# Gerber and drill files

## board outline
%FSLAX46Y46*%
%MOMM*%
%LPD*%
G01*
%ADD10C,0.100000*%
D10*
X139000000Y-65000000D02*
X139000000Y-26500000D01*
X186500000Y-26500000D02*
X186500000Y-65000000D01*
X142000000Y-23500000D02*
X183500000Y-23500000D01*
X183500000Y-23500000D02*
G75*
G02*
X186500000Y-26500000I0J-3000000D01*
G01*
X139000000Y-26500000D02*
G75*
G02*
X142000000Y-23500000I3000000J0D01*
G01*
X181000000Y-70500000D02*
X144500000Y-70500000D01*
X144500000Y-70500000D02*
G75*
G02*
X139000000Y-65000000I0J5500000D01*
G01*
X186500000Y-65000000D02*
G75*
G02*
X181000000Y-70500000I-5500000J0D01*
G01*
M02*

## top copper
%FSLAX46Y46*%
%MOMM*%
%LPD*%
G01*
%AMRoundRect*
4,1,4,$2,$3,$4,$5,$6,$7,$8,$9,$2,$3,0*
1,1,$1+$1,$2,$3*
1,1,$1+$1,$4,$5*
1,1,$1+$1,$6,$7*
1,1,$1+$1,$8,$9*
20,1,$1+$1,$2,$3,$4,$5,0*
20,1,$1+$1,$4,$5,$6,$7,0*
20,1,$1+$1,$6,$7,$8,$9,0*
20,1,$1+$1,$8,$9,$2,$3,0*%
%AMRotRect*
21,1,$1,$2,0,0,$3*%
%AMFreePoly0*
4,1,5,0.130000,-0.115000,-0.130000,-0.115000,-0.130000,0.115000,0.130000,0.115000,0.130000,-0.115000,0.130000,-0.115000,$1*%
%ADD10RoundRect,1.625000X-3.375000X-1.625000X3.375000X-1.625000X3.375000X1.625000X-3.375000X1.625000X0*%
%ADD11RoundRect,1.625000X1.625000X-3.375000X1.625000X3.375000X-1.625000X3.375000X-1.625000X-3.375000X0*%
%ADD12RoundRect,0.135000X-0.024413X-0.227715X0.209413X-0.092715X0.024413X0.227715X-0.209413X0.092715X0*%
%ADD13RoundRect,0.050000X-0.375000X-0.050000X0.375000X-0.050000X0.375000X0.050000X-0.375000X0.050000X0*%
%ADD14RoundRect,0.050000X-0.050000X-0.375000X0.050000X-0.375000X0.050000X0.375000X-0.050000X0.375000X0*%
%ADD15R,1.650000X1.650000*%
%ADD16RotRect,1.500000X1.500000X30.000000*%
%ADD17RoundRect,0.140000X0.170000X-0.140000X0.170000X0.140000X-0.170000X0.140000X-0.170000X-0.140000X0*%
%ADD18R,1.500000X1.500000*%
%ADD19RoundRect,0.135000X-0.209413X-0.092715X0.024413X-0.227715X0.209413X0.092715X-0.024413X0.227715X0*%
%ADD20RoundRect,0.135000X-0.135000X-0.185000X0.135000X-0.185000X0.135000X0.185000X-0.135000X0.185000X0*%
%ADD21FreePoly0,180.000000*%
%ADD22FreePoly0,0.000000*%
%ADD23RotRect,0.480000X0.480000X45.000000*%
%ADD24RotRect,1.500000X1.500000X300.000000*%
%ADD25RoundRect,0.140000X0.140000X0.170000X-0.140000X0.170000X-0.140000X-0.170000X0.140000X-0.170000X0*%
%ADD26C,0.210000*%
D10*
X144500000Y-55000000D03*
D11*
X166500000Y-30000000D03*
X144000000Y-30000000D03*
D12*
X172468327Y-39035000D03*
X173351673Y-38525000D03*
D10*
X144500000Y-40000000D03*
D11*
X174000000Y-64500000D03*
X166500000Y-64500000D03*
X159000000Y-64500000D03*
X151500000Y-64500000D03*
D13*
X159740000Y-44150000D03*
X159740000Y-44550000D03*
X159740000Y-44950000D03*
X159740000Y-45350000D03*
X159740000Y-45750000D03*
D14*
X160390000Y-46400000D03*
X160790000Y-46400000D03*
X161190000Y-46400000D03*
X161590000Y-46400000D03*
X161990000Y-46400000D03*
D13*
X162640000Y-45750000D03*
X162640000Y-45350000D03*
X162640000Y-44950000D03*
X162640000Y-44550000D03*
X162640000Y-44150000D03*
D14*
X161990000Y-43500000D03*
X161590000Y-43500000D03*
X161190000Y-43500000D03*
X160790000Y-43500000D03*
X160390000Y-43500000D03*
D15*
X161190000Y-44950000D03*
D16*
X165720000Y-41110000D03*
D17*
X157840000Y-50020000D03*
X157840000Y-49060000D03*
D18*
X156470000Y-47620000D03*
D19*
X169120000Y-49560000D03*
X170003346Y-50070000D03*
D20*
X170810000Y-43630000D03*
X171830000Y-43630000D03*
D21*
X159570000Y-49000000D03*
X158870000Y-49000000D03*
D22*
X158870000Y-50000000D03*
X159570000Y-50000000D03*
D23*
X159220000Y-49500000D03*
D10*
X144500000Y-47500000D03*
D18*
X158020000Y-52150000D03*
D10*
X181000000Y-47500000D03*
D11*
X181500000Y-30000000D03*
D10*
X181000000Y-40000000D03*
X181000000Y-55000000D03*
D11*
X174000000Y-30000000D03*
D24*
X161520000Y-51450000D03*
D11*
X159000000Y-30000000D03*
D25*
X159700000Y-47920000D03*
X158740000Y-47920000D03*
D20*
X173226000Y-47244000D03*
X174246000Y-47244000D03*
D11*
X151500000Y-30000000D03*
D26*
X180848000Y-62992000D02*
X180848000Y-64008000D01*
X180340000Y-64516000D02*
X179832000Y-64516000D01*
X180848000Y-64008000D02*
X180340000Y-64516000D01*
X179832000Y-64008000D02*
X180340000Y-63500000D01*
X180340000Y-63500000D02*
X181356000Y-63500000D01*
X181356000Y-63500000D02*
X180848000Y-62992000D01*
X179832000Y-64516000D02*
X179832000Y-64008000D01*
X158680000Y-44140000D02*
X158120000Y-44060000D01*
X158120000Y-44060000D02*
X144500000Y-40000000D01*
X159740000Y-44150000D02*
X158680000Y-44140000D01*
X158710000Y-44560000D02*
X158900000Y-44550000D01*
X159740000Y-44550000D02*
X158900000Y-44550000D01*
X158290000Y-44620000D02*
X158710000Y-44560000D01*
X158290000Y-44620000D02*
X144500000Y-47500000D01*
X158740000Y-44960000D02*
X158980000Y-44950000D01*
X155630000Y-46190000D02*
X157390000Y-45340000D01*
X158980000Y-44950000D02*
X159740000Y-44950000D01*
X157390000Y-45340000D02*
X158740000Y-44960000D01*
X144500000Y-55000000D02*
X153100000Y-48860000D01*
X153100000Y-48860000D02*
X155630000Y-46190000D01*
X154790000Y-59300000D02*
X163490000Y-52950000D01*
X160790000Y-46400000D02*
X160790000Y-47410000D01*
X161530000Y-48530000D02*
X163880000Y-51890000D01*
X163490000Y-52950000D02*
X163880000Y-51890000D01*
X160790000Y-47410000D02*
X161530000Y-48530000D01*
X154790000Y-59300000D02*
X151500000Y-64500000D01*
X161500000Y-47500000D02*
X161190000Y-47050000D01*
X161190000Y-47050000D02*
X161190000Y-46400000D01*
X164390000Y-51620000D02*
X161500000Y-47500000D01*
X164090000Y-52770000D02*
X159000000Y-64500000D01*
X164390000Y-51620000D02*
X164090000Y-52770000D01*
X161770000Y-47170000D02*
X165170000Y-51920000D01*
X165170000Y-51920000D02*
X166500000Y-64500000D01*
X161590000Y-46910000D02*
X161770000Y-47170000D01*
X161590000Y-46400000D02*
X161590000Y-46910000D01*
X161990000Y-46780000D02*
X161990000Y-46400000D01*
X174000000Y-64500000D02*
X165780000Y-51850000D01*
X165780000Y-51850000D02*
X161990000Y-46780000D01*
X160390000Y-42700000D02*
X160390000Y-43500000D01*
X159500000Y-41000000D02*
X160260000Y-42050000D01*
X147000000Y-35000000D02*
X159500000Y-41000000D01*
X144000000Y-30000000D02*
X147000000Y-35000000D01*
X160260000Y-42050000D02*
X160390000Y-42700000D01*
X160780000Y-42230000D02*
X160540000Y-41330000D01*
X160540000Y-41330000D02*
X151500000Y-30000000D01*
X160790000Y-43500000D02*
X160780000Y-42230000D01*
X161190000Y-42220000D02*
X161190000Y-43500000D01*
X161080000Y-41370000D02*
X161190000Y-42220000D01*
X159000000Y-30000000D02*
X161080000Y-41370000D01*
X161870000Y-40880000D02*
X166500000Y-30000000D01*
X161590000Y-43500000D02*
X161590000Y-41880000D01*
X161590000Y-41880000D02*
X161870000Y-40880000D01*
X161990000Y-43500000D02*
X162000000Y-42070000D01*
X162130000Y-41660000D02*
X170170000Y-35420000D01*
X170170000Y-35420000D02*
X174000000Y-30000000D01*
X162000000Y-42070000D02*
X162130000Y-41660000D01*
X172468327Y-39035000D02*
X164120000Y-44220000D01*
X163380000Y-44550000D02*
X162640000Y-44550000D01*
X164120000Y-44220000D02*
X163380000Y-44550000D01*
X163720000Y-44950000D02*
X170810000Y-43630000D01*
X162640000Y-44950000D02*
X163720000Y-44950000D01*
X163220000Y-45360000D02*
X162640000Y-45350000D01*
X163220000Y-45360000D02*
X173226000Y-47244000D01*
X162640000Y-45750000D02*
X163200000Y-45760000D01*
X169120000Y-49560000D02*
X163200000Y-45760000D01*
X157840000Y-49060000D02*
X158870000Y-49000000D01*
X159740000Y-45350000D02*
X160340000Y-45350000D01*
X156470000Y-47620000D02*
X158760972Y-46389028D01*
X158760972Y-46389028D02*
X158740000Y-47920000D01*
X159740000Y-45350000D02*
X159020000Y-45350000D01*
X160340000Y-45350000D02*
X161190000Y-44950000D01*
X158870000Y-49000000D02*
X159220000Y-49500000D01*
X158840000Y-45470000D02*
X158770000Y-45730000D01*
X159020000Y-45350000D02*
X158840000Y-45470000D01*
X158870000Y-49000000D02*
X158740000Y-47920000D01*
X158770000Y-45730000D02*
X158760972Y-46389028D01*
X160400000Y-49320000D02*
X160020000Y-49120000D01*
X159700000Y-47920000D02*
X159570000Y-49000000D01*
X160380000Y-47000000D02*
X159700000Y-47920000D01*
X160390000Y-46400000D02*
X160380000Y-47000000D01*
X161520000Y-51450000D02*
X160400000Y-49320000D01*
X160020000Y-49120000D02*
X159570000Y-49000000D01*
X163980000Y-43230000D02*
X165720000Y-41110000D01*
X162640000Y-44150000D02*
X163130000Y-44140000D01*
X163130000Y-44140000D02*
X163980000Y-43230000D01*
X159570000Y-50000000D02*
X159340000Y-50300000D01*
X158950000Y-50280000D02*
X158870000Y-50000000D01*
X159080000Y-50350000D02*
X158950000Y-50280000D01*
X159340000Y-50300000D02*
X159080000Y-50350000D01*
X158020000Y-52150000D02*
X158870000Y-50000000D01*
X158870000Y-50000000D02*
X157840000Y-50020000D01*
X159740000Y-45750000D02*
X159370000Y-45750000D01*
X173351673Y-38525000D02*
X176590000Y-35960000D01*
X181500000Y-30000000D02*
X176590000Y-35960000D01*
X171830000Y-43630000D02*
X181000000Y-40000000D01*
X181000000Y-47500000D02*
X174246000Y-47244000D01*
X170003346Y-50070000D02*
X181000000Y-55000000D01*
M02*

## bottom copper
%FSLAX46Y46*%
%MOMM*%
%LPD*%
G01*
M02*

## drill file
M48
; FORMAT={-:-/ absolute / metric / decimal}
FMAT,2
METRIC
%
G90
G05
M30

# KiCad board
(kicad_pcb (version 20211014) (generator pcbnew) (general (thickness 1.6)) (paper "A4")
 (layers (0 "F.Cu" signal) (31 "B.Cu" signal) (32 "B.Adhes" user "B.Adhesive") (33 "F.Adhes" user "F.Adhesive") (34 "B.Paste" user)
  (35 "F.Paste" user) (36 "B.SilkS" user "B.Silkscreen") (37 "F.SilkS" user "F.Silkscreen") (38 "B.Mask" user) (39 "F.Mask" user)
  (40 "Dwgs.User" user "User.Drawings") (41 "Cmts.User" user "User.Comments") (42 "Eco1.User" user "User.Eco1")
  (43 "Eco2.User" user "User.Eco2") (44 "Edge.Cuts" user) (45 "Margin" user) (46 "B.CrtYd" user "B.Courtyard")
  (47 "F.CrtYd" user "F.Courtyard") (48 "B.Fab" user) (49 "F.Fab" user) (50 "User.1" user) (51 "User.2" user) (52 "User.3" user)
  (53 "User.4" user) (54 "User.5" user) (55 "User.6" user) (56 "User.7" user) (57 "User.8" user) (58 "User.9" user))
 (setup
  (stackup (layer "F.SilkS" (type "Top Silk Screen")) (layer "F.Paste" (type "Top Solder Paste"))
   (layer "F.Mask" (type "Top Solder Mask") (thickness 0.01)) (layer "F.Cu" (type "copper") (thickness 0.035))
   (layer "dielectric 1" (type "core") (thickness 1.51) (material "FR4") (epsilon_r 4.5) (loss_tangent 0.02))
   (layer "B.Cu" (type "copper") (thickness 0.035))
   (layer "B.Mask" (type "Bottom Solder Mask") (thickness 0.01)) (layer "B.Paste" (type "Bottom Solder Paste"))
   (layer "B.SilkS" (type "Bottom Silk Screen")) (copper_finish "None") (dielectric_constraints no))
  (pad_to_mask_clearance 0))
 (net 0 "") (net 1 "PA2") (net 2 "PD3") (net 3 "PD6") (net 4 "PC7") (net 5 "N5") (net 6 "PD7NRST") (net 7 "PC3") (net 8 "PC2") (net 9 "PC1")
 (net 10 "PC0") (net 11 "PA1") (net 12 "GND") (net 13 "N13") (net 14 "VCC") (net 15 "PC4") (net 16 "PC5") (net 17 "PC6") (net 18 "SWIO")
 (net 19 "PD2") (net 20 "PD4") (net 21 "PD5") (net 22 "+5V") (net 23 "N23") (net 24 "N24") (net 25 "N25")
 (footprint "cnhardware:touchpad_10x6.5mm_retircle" (layer "F.Cu") (at 144.5 55)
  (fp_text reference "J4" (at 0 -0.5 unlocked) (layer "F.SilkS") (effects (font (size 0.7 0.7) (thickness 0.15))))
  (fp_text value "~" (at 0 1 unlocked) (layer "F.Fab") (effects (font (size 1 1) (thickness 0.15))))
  (pad "1" smd roundrect (at 0 0) (size 10 6.5) (layers "F.Cu") (roundrect_rratio 0.25) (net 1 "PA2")))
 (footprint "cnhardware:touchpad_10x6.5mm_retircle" (layer "F.Cu") (at 166.5 30 90)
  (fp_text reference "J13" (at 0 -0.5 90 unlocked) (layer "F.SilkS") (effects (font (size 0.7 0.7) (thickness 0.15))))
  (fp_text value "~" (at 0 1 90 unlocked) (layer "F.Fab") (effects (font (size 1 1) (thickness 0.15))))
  (pad "1" smd roundrect (at 0 0 90) (size 10 6.5) (layers "F.Cu") (roundrect_rratio 0.25) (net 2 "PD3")))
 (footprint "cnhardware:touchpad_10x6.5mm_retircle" (layer "F.Cu") (at 144 30 90)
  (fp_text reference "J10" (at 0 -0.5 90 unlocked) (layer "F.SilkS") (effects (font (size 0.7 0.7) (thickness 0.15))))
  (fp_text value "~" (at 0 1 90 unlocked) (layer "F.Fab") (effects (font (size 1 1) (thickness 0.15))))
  (pad "1" smd roundrect (at 0 0 90) (size 10 6.5) (layers "F.Cu") (roundrect_rratio 0.25) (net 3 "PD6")))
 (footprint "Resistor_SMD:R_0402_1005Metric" (layer "F.Cu") (at 172.91 38.78 30)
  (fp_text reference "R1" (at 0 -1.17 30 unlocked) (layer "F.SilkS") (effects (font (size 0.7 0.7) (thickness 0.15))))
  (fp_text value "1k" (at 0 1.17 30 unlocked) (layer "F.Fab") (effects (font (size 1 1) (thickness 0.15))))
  (pad "1" smd roundrect (at -0.51 0 30) (size 0.54 0.64) (layers "F.Cu" "F.Paste" "F.Mask") (roundrect_rratio 0.25) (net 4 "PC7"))
  (pad "2" smd roundrect (at 0.51 0 30) (size 0.54 0.64) (layers "F.Cu" "F.Paste" "F.Mask") (roundrect_rratio 0.25) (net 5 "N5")))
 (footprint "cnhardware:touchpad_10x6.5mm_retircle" (layer "F.Cu") (at 144.5 40)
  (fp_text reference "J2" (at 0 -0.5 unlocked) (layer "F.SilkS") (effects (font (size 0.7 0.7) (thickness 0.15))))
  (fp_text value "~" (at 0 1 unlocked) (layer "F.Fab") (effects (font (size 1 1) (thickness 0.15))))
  (pad "1" smd roundrect (at 0 0) (size 10 6.5) (layers "F.Cu") (roundrect_rratio 0.25) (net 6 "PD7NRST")))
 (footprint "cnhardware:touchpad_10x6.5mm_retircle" (layer "F.Cu") (at 174 64.5 90)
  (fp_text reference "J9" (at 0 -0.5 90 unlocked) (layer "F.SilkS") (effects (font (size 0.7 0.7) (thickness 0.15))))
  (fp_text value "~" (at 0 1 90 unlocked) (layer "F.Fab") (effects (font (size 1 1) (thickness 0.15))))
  (pad "1" smd roundrect (at 0 0 90) (size 10 6.5) (layers "F.Cu") (roundrect_rratio 0.25) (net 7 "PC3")))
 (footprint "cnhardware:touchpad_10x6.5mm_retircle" (layer "F.Cu") (at 166.5 64.5 90)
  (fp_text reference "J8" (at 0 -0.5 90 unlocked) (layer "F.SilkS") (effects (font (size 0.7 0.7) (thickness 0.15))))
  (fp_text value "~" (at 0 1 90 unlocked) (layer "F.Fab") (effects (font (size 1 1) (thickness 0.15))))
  (pad "1" smd roundrect (at 0 0 90) (size 10 6.5) (layers "F.Cu") (roundrect_rratio 0.25) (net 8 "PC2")))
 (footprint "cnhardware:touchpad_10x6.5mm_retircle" (layer "F.Cu") (at 159 64.5 90)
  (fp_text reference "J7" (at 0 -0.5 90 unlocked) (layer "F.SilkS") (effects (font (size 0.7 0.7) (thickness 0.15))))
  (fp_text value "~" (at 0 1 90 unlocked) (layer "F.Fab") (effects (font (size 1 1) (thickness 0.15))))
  (pad "1" smd roundrect (at 0 0 90) (size 10 6.5) (layers "F.Cu") (roundrect_rratio 0.25) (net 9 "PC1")))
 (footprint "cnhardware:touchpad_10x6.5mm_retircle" (layer "F.Cu") (at 151.5 64.5 90)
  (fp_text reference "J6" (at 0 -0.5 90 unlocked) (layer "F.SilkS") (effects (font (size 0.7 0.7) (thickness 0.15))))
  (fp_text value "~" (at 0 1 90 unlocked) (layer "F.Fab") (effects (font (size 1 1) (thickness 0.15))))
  (pad "1" smd roundrect (at 0 0 90) (size 10 6.5) (layers "F.Cu") (roundrect_rratio 0.25) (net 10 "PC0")))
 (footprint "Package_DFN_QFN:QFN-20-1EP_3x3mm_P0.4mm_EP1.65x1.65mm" (layer "F.Cu") (at 161.19 44.95)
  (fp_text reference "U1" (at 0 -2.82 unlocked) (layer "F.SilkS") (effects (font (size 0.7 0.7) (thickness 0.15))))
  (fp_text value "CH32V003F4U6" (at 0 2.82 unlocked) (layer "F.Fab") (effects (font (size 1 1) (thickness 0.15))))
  (pad "" smd roundrect (at 0.41 -0.41) (size 0.67 0.67) (layers "F.Paste") (roundrect_rratio 0.25))
  (pad "" smd roundrect (at -0.41 0.41) (size 0.67 0.67) (layers "F.Paste") (roundrect_rratio 0.25))
  (pad "" smd roundrect (at 0.41 0.41) (size 0.67 0.67) (layers "F.Paste") (roundrect_rratio 0.25))
  (pad "" smd roundrect (at -0.41 -0.41) (size 0.67 0.67) (layers "F.Paste") (roundrect_rratio 0.25))
  (pad "1" smd roundrect (at -1.45 -0.8) (size 0.85 0.2) (layers "F.Cu" "F.Paste" "F.Mask") (roundrect_rratio 0.25) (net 6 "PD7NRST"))
  (pad "2" smd roundrect (at -1.45 -0.4) (size 0.85 0.2) (layers "F.Cu" "F.Paste" "F.Mask") (roundrect_rratio 0.25) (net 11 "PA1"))
  (pad "3" smd roundrect (at -1.45 0) (size 0.85 0.2) (layers "F.Cu" "F.Paste" "F.Mask") (roundrect_rratio 0.25) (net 1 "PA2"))
  (pad "4" smd roundrect (at -1.45 0.4) (size 0.85 0.2) (layers "F.Cu" "F.Paste" "F.Mask") (roundrect_rratio 0.25) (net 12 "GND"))
  (pad "5" smd roundrect (at -1.45 0.8) (size 0.85 0.2) (layers "F.Cu" "F.Paste" "F.Mask") (roundrect_rratio 0.25) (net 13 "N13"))
  (pad "6" smd roundrect (at -0.8 1.45) (size 0.2 0.85) (layers "F.Cu" "F.Paste" "F.Mask") (roundrect_rratio 0.25) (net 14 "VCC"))
  (pad "7" smd roundrect (at -0.4 1.45) (size 0.2 0.85) (layers "F.Cu" "F.Paste" "F.Mask") (roundrect_rratio 0.25) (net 10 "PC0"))
  (pad "8" smd roundrect (at 0 1.45) (size 0.2 0.85) (layers "F.Cu" "F.Paste" "F.Mask") (roundrect_rratio 0.25) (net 9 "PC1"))
  (pad "9" smd roundrect (at 0.4 1.45) (size 0.2 0.85) (layers "F.Cu" "F.Paste" "F.Mask") (roundrect_rratio 0.25) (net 8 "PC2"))
  (pad "10" smd roundrect (at 0.8 1.45) (size 0.2 0.85) (layers "F.Cu" "F.Paste" "F.Mask") (roundrect_rratio 0.25) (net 7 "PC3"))
  (pad "11" smd roundrect (at 1.45 0.8) (size 0.85 0.2) (layers "F.Cu" "F.Paste" "F.Mask") (roundrect_rratio 0.25) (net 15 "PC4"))
  (pad "12" smd roundrect (at 1.45 0.4) (size 0.85 0.2) (layers "F.Cu" "F.Paste" "F.Mask") (roundrect_rratio 0.25) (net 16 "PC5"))
  (pad "13" smd roundrect (at 1.45 0) (size 0.85 0.2) (layers "F.Cu" "F.Paste" "F.Mask") (roundrect_rratio 0.25) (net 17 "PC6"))
  (pad "14" smd roundrect (at 1.45 -0.4) (size 0.85 0.2) (layers "F.Cu" "F.Paste" "F.Mask") (roundrect_rratio 0.25) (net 4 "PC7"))
  (pad "15" smd roundrect (at 1.45 -0.8) (size 0.85 0.2) (layers "F.Cu" "F.Paste" "F.Mask") (roundrect_rratio 0.25) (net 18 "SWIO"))
  (pad "16" smd roundrect (at 0.8 -1.45) (size 0.2 0.85) (layers "F.Cu" "F.Paste" "F.Mask") (roundrect_rratio 0.25) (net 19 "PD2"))
  (pad "17" smd roundrect (at 0.4 -1.45) (size 0.2 0.85) (layers "F.Cu" "F.Paste" "F.Mask") (roundrect_rratio 0.25) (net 2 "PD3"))
  (pad "18" smd roundrect (at 0 -1.45) (size 0.2 0.85) (layers "F.Cu" "F.Paste" "F.Mask") (roundrect_rratio 0.25) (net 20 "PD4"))
  (pad "19" smd roundrect (at -0.4 -1.45) (size 0.2 0.85) (layers "F.Cu" "F.Paste" "F.Mask") (roundrect_rratio 0.25) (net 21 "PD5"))
  (pad "20" smd roundrect (at -0.8 -1.45) (size 0.2 0.85) (layers "F.Cu" "F.Paste" "F.Mask") (roundrect_rratio 0.25) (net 3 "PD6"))
  (pad "21" smd rect (at 0 0) (size 1.65 1.65) (layers "F.Cu" "F.Mask") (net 12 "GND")))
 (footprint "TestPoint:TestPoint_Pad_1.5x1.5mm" (layer "F.Cu") (at 165.72 41.11 30)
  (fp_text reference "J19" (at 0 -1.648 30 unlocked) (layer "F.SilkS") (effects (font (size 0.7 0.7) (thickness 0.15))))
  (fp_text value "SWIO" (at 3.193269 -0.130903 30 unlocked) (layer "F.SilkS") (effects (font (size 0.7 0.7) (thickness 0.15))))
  (pad "1" smd rect (at 0 0 30) (size 1.5 1.5) (layers "F.Cu" "F.Mask") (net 18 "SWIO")))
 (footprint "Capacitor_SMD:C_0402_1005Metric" (layer "F.Cu") (at 157.84 49.54 90)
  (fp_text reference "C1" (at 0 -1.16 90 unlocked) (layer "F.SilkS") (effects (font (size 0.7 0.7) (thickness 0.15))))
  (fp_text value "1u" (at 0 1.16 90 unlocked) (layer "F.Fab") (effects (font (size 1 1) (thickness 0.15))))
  (pad "1" smd roundrect (at -0.48 0 90) (size 0.56 0.62) (layers "F.Cu" "F.Paste" "F.Mask") (roundrect_rratio 0.25) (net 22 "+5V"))
  (pad "2" smd roundrect (at 0.48 0 90) (size 0.56 0.62) (layers "F.Cu" "F.Paste" "F.Mask") (roundrect_rratio 0.25) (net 12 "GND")))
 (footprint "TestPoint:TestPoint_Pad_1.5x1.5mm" (layer "F.Cu") (at 156.47 47.62)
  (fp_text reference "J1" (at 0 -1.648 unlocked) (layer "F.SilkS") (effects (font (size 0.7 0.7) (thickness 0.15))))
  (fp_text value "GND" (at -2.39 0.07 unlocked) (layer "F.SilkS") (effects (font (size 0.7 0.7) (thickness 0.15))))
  (pad "1" smd rect (at 0 0) (size 1.5 1.5) (layers "F.Cu" "F.Mask") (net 12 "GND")))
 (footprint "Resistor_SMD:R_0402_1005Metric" (layer "F.Cu") (at 169.561673 49.815 -30)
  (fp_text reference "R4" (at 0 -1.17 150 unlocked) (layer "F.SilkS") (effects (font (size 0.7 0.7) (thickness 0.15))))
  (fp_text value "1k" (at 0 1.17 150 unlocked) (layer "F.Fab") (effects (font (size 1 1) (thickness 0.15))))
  (pad "1" smd roundrect (at -0.51 0 330) (size 0.54 0.64) (layers "F.Cu" "F.Paste" "F.Mask") (roundrect_rratio 0.25) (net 15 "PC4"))
  (pad "2" smd roundrect (at 0.51 0 330) (size 0.54 0.64) (layers "F.Cu" "F.Paste" "F.Mask") (roundrect_rratio 0.25) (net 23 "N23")))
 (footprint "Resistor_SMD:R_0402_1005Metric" (layer "F.Cu") (at 171.32 43.63)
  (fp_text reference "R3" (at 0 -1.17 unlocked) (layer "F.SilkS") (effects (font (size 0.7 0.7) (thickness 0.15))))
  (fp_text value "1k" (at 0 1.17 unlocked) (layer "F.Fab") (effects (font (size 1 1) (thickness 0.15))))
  (pad "1" smd roundrect (at -0.51 0) (size 0.54 0.64) (layers "F.Cu" "F.Paste" "F.Mask") (roundrect_rratio 0.25) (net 17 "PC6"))
  (pad "2" smd roundrect (at 0.51 0) (size 0.54 0.64) (layers "F.Cu" "F.Paste" "F.Mask") (roundrect_rratio 0.25) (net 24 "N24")))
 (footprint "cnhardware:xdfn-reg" (layer "F.Cu") (at 159.22 49.5 180)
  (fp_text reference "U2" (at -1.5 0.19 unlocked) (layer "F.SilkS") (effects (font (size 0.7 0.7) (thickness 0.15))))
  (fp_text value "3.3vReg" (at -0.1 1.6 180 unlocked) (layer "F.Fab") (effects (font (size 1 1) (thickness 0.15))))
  (pad "1" smd custom (at -0.35 0.5 180) (size 0.26 0.23) (layers "F.Cu" "F.Paste" "F.Mask") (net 14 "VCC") (zone_connect 0)
   (options (clearance outline) (anchor rect)) (primitives))
  (pad "2" smd custom (at 0.35 0.5 180) (size 0.26 0.23) (layers "F.Cu" "F.Paste" "F.Mask") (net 12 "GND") (zone_connect 0)
   (options (clearance outline) (anchor rect)) (primitives))
  (pad "3" smd custom (at 0.35 -0.5) (size 0.26 0.23) (layers "F.Cu" "F.Paste" "F.Mask") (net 22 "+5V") (zone_connect 0)
   (options (clearance outline) (anchor rect)) (primitives))
  (pad "4" smd custom (at -0.35 -0.5) (size 0.26 0.23) (layers "F.Cu" "F.Paste" "F.Mask") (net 22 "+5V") (zone_connect 0)
   (options (clearance outline) (anchor rect)) (primitives))
  (pad "5" smd rect (at 0 0 45) (size 0.48 0.48) (layers "F.Cu" "F.Paste" "F.Mask") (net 12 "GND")))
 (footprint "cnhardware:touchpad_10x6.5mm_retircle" (layer "F.Cu") (at 144.5 47.5)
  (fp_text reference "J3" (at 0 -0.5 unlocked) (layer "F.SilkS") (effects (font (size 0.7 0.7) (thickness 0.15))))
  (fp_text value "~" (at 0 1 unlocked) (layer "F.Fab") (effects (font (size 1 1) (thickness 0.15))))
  (pad "1" smd roundrect (at 0 0) (size 10 6.5) (layers "F.Cu") (roundrect_rratio 0.25) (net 11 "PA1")))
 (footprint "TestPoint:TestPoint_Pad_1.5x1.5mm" (layer "F.Cu") (at 158.02 52.15 90)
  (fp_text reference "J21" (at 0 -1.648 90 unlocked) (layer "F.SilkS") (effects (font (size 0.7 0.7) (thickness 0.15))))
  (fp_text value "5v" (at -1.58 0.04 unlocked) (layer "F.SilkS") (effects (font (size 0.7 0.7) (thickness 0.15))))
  (pad "1" smd rect (at 0 0 90) (size 1.5 1.5) (layers "F.Cu" "F.Mask") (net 22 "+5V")))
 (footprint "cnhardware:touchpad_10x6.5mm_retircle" (layer "F.Cu") (at 181 47.5)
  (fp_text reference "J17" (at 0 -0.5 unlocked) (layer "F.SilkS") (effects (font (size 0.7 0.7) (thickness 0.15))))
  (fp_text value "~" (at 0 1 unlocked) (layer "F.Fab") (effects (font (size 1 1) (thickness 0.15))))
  (pad "1" smd roundrect (at 0 0) (size 10 6.5) (layers "F.Cu") (roundrect_rratio 0.25) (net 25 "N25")))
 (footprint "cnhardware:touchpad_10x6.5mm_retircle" (layer "F.Cu") (at 181.5 30 90)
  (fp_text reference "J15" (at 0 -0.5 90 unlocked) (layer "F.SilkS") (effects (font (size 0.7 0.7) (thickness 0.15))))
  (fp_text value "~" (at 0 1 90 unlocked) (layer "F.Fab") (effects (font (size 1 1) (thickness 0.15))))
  (pad "1" smd roundrect (at 0 0 90) (size 10 6.5) (layers "F.Cu") (roundrect_rratio 0.25) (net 5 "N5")))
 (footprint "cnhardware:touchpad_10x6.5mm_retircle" (layer "F.Cu") (at 181 40)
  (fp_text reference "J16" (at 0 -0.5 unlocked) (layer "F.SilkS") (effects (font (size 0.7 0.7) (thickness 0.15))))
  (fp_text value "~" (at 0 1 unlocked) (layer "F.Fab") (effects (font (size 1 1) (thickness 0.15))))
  (pad "1" smd roundrect (at 0 0) (size 10 6.5) (layers "F.Cu") (roundrect_rratio 0.25) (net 24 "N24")))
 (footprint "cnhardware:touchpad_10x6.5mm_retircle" (layer "F.Cu") (at 181 55)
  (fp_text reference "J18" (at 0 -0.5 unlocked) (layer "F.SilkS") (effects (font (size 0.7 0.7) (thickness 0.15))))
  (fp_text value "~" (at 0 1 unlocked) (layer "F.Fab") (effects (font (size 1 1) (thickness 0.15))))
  (pad "1" smd roundrect (at 0 0) (size 10 6.5) (layers "F.Cu") (roundrect_rratio 0.25) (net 23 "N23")))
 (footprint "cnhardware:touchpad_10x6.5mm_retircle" (layer "F.Cu") (at 174 30 90)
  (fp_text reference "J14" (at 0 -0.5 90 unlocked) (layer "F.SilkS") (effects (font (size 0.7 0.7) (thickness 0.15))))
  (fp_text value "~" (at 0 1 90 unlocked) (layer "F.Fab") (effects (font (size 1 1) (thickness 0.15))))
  (pad "1" smd roundrect (at 0 0 90) (size 10 6.5) (layers "F.Cu") (roundrect_rratio 0.25) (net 19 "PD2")))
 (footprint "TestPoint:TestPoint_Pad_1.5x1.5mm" (layer "F.Cu") (at 161.52 51.45 -60)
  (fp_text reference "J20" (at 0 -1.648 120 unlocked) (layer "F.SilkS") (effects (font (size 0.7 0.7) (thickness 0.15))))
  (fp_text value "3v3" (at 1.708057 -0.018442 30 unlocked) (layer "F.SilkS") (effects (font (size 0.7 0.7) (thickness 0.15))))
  (pad "1" smd rect (at 0 0 300) (size 1.5 1.5) (layers "F.Cu" "F.Mask") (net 14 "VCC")))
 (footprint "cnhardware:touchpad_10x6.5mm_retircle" (layer "F.Cu") (at 159 30 90)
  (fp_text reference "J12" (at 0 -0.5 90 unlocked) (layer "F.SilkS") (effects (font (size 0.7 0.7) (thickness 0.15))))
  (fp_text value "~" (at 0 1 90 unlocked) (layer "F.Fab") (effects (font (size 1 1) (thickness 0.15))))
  (pad "1" smd roundrect (at 0 0 90) (size 10 6.5) (layers "F.Cu") (roundrect_rratio 0.25) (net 20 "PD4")))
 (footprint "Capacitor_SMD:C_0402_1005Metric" (layer "F.Cu") (at 159.22 47.92 180)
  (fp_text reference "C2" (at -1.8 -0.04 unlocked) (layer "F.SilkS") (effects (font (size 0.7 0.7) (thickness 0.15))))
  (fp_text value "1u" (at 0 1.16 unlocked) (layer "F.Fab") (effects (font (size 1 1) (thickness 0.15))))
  (pad "1" smd roundrect (at -0.48 0 180) (size 0.56 0.62) (layers "F.Cu" "F.Paste" "F.Mask") (roundrect_rratio 0.25) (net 14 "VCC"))
  (pad "2" smd roundrect (at 0.48 0 180) (size 0.56 0.62) (layers "F.Cu" "F.Paste" "F.Mask") (roundrect_rratio 0.25) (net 12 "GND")))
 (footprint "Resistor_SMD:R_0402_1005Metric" (layer "F.Cu") (at 173.736 47.244)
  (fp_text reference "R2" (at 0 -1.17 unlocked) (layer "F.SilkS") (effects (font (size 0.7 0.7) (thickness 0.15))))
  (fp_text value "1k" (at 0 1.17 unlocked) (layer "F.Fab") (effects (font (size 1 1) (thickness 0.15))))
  (pad "1" smd roundrect (at -0.51 0) (size 0.54 0.64) (layers "F.Cu" "F.Paste" "F.Mask") (roundrect_rratio 0.25) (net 16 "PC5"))
  (pad "2" smd roundrect (at 0.51 0) (size 0.54 0.64) (layers "F.Cu" "F.Paste" "F.Mask") (roundrect_rratio 0.25) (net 25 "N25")))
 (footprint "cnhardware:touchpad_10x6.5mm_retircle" (layer "F.Cu") (at 151.5 30 90)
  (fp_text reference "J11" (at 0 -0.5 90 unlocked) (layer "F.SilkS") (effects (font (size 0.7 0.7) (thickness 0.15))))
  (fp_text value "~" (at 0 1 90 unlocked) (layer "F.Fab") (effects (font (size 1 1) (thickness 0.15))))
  (pad "1" smd roundrect (at 0 0 90) (size 10 6.5) (layers "F.Cu") (roundrect_rratio 0.25) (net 21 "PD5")))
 (gr_line (start 139 65) (end 139 26.5) (layer "Edge.Cuts") (width 0.1))
 (gr_line (start 186.5 26.5) (end 186.5 65) (layer "Edge.Cuts") (width 0.1))
 (gr_line (start 142 23.5) (end 183.5 23.5) (layer "Edge.Cuts") (width 0.1))
 (gr_arc (start 183.5 23.5) (mid 185.62132 24.37868) (end 186.5 26.5) (layer "Edge.Cuts") (width 0.1))
 (gr_arc (start 139 26.5) (mid 139.87868 24.37868) (end 142 23.5) (layer "Edge.Cuts") (width 0.1))
 (gr_line (start 181 70.5) (end 144.5 70.5) (layer "Edge.Cuts") (width 0.1))
 (gr_arc (start 144.5 70.5) (mid 140.610913 68.889087) (end 139 65) (layer "Edge.Cuts") (width 0.1))
 (gr_arc (start 186.5 65) (mid 184.889087 68.889087) (end 181 70.5) (layer "Edge.Cuts") (width 0.1))
 (segment (start 180.848 62.992) (end 180.848 64.008) (width 0.21) (layer "F.Cu") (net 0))
 (segment (start 180.34 64.516) (end 179.832 64.516) (width 0.21) (layer "F.Cu") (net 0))
 (segment (start 180.848 64.008) (end 180.34 64.516) (width 0.21) (layer "F.Cu") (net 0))
 (segment (start 179.832 64.008) (end 180.34 63.5) (width 0.21) (layer "F.Cu") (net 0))
 (segment (start 180.34 63.5) (end 181.356 63.5) (width 0.21) (layer "F.Cu") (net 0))
 (segment (start 181.356 63.5) (end 180.848 62.992) (width 0.21) (layer "F.Cu") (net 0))
 (segment (start 179.832 64.516) (end 179.832 64.008) (width 0.21) (layer "F.Cu") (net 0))
 (segment (start 158.68 44.14) (end 158.12 44.06) (width 0.21) (layer "F.Cu") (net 6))
 (segment (start 158.12 44.06) (end 144.5 40) (width 0.21) (layer "F.Cu") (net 6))
 (segment (start 159.74 44.15) (end 158.68 44.14) (width 0.21) (layer "F.Cu") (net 6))
 (segment (start 158.71 44.56) (end 158.9 44.55) (width 0.21) (layer "F.Cu") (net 11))
 (segment (start 159.74 44.55) (end 158.9 44.55) (width 0.21) (layer "F.Cu") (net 11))
 (segment (start 158.29 44.62) (end 158.71 44.56) (width 0.21) (layer "F.Cu") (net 11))
 (segment (start 158.29 44.62) (end 144.5 47.5) (width 0.21) (layer "F.Cu") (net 11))
 (segment (start 158.74 44.96) (end 158.98 44.95) (width 0.21) (layer "F.Cu") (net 1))
 (segment (start 155.63 46.19) (end 157.39 45.34) (width 0.21) (layer "F.Cu") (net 1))
 (segment (start 158.98 44.95) (end 159.74 44.95) (width 0.21) (layer "F.Cu") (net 1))
 (segment (start 157.39 45.34) (end 158.74 44.96) (width 0.21) (layer "F.Cu") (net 1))
 (segment (start 144.5 55) (end 153.1 48.86) (width 0.21) (layer "F.Cu") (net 1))
 (segment (start 153.1 48.86) (end 155.63 46.19) (width 0.21) (layer "F.Cu") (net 1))
 (segment (start 154.79 59.3) (end 163.49 52.95) (width 0.21) (layer "F.Cu") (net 10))
 (segment (start 160.79 46.4) (end 160.79 47.41) (width 0.21) (layer "F.Cu") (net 10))
 (segment (start 161.53 48.53) (end 163.88 51.89) (width 0.21) (layer "F.Cu") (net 10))
 (segment (start 163.49 52.95) (end 163.88 51.89) (width 0.21) (layer "F.Cu") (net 10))
 (segment (start 160.79 47.41) (end 161.53 48.53) (width 0.21) (layer "F.Cu") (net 10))
 (segment (start 154.79 59.3) (end 151.5 64.5) (width 0.21) (layer "F.Cu") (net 10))
 (segment (start 161.5 47.5) (end 161.19 47.05) (width 0.21) (layer "F.Cu") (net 9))
 (segment (start 161.19 47.05) (end 161.19 46.4) (width 0.21) (layer "F.Cu") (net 9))
 (segment (start 164.39 51.62) (end 161.5 47.5) (width 0.21) (layer "F.Cu") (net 9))
 (segment (start 164.09 52.77) (end 159 64.5) (width 0.21) (layer "F.Cu") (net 9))
 (segment (start 164.39 51.62) (end 164.09 52.77) (width 0.21) (layer "F.Cu") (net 9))
 (segment (start 161.77 47.17) (end 165.17 51.92) (width 0.21) (layer "F.Cu") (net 8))
 (segment (start 165.17 51.92) (end 166.5 64.5) (width 0.21) (layer "F.Cu") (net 8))
 (segment (start 161.59 46.91) (end 161.77 47.17) (width 0.21) (layer "F.Cu") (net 8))
 (segment (start 161.59 46.4) (end 161.59 46.91) (width 0.21) (layer "F.Cu") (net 8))
 (segment (start 161.99 46.78) (end 161.99 46.4) (width 0.21) (layer "F.Cu") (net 7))
 (segment (start 174 64.5) (end 165.78 51.85) (width 0.21) (layer "F.Cu") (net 7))
 (segment (start 165.78 51.85) (end 161.99 46.78) (width 0.21) (layer "F.Cu") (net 7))
 (segment (start 160.39 42.7) (end 160.39 43.5) (width 0.21) (layer "F.Cu") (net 3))
 (segment (start 159.5 41) (end 160.26 42.05) (width 0.21) (layer "F.Cu") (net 3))
 (segment (start 147 35) (end 159.5 41) (width 0.21) (layer "F.Cu") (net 3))
 (segment (start 144 30) (end 147 35) (width 0.21) (layer "F.Cu") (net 3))
 (segment (start 160.26 42.05) (end 160.39 42.7) (width 0.21) (layer "F.Cu") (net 3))
 (segment (start 160.78 42.23) (end 160.54 41.33) (width 0.21) (layer "F.Cu") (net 21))
 (segment (start 160.54 41.33) (end 151.5 30) (width 0.21) (layer "F.Cu") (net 21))
 (segment (start 160.79 43.5) (end 160.78 42.23) (width 0.21) (layer "F.Cu") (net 21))
 (segment (start 161.19 42.22) (end 161.19 43.5) (width 0.21) (layer "F.Cu") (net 20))
 (segment (start 161.08 41.37) (end 161.19 42.22) (width 0.21) (layer "F.Cu") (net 20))
 (segment (start 159 30) (end 161.08 41.37) (width 0.21) (layer "F.Cu") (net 20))
 (segment (start 161.87 40.88) (end 166.5 30) (width 0.21) (layer "F.Cu") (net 2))
 (segment (start 161.59 43.5) (end 161.59 41.88) (width 0.21) (layer "F.Cu") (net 2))
 (segment (start 161.59 41.88) (end 161.87 40.88) (width 0.21) (layer "F.Cu") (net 2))
 (segment (start 161.99 43.5) (end 162 42.07) (width 0.21) (layer "F.Cu") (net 19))
 (segment (start 162.13 41.66) (end 170.17 35.42) (width 0.21) (layer "F.Cu") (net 19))
 (segment (start 170.17 35.42) (end 174 30) (width 0.21) (layer "F.Cu") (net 19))
 (segment (start 162 42.07) (end 162.13 41.66) (width 0.21) (layer "F.Cu") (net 19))
 (segment (start 172.468327 39.035) (end 164.12 44.22) (width 0.21) (layer "F.Cu") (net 4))
 (segment (start 163.38 44.55) (end 162.64 44.55) (width 0.21) (layer "F.Cu") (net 4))
 (segment (start 164.12 44.22) (end 163.38 44.55) (width 0.21) (layer "F.Cu") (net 4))
 (segment (start 163.72 44.95) (end 170.81 43.63) (width 0.21) (layer "F.Cu") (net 17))
 (segment (start 162.64 44.95) (end 163.72 44.95) (width 0.21) (layer "F.Cu") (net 17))
 (segment (start 163.22 45.36) (end 162.64 45.35) (width 0.21) (layer "F.Cu") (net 16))
 (segment (start 163.22 45.36) (end 173.226 47.244) (width 0.21) (layer "F.Cu") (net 16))
 (segment (start 162.64 45.75) (end 163.2 45.76) (width 0.21) (layer "F.Cu") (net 15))
 (segment (start 169.12 49.56) (end 163.2 45.76) (width 0.21) (layer "F.Cu") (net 15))
 (segment (start 157.84 49.06) (end 158.87 49) (width 0.21) (layer "F.Cu") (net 12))
 (segment (start 159.74 45.35) (end 160.34 45.35) (width 0.21) (layer "F.Cu") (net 12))
 (segment (start 156.47 47.62) (end 158.760972 46.389028) (width 0.21) (layer "F.Cu") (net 12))
 (segment (start 158.760972 46.389028) (end 158.74 47.92) (width 0.21) (layer "F.Cu") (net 12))
 (segment (start 159.74 45.35) (end 159.02 45.35) (width 0.21) (layer "F.Cu") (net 12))
 (segment (start 160.34 45.35) (end 161.19 44.95) (width 0.21) (layer "F.Cu") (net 12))
 (segment (start 158.87 49) (end 159.22 49.5) (width 0.21) (layer "F.Cu") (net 12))
 (segment (start 158.84 45.47) (end 158.77 45.73) (width 0.21) (layer "F.Cu") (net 12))
 (segment (start 159.02 45.35) (end 158.84 45.47) (width 0.21) (layer "F.Cu") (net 12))
 (segment (start 158.87 49) (end 158.74 47.92) (width 0.21) (layer "F.Cu") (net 12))
 (segment (start 158.77 45.73) (end 158.760972 46.389028) (width 0.21) (layer "F.Cu") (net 12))
 (segment (start 160.4 49.32) (end 160.02 49.12) (width 0.21) (layer "F.Cu") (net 14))
 (segment (start 159.7 47.92) (end 159.57 49) (width 0.21) (layer "F.Cu") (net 14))
 (segment (start 160.38 47) (end 159.7 47.92) (width 0.21) (layer "F.Cu") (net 14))
 (segment (start 160.39 46.4) (end 160.38 47) (width 0.21) (layer "F.Cu") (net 14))
 (segment (start 161.52 51.45) (end 160.4 49.32) (width 0.21) (layer "F.Cu") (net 14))
 (segment (start 160.02 49.12) (end 159.57 49) (width 0.21) (layer "F.Cu") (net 14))
 (segment (start 163.98 43.23) (end 165.72 41.11) (width 0.21) (layer "F.Cu") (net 18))
 (segment (start 162.64 44.15) (end 163.13 44.14) (width 0.21) (layer "F.Cu") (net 18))
 (segment (start 163.13 44.14) (end 163.98 43.23) (width 0.21) (layer "F.Cu") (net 18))
 (segment (start 159.57 50) (end 159.34 50.3) (width 0.21) (layer "F.Cu") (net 22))
 (segment (start 158.95 50.28) (end 158.87 50) (width 0.21) (layer "F.Cu") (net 22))
 (segment (start 159.08 50.35) (end 158.95 50.28) (width 0.21) (layer "F.Cu") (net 22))
 (segment (start 159.34 50.3) (end 159.08 50.35) (width 0.21) (layer "F.Cu") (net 22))
 (segment (start 158.02 52.15) (end 158.87 50) (width 0.21) (layer "F.Cu") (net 22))
 (segment (start 158.87 50) (end 157.84 50.02) (width 0.21) (layer "F.Cu") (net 22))
 (segment (start 159.74 45.75) (end 159.37 45.75) (width 0.21) (layer "F.Cu") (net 13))
 (segment (start 173.351673 38.525) (end 176.59 35.96) (width 0.21) (layer "F.Cu") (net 5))
 (segment (start 181.5 30) (end 176.59 35.96) (width 0.21) (layer "F.Cu") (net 5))
 (segment (start 171.83 43.63) (end 181 40) (width 0.21) (layer "F.Cu") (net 24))
 (segment (start 181 47.5) (end 174.246 47.244) (width 0.21) (layer "F.Cu") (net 25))
 (segment (start 170.003346 50.07) (end 181 55) (width 0.21) (layer "F.Cu") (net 23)))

